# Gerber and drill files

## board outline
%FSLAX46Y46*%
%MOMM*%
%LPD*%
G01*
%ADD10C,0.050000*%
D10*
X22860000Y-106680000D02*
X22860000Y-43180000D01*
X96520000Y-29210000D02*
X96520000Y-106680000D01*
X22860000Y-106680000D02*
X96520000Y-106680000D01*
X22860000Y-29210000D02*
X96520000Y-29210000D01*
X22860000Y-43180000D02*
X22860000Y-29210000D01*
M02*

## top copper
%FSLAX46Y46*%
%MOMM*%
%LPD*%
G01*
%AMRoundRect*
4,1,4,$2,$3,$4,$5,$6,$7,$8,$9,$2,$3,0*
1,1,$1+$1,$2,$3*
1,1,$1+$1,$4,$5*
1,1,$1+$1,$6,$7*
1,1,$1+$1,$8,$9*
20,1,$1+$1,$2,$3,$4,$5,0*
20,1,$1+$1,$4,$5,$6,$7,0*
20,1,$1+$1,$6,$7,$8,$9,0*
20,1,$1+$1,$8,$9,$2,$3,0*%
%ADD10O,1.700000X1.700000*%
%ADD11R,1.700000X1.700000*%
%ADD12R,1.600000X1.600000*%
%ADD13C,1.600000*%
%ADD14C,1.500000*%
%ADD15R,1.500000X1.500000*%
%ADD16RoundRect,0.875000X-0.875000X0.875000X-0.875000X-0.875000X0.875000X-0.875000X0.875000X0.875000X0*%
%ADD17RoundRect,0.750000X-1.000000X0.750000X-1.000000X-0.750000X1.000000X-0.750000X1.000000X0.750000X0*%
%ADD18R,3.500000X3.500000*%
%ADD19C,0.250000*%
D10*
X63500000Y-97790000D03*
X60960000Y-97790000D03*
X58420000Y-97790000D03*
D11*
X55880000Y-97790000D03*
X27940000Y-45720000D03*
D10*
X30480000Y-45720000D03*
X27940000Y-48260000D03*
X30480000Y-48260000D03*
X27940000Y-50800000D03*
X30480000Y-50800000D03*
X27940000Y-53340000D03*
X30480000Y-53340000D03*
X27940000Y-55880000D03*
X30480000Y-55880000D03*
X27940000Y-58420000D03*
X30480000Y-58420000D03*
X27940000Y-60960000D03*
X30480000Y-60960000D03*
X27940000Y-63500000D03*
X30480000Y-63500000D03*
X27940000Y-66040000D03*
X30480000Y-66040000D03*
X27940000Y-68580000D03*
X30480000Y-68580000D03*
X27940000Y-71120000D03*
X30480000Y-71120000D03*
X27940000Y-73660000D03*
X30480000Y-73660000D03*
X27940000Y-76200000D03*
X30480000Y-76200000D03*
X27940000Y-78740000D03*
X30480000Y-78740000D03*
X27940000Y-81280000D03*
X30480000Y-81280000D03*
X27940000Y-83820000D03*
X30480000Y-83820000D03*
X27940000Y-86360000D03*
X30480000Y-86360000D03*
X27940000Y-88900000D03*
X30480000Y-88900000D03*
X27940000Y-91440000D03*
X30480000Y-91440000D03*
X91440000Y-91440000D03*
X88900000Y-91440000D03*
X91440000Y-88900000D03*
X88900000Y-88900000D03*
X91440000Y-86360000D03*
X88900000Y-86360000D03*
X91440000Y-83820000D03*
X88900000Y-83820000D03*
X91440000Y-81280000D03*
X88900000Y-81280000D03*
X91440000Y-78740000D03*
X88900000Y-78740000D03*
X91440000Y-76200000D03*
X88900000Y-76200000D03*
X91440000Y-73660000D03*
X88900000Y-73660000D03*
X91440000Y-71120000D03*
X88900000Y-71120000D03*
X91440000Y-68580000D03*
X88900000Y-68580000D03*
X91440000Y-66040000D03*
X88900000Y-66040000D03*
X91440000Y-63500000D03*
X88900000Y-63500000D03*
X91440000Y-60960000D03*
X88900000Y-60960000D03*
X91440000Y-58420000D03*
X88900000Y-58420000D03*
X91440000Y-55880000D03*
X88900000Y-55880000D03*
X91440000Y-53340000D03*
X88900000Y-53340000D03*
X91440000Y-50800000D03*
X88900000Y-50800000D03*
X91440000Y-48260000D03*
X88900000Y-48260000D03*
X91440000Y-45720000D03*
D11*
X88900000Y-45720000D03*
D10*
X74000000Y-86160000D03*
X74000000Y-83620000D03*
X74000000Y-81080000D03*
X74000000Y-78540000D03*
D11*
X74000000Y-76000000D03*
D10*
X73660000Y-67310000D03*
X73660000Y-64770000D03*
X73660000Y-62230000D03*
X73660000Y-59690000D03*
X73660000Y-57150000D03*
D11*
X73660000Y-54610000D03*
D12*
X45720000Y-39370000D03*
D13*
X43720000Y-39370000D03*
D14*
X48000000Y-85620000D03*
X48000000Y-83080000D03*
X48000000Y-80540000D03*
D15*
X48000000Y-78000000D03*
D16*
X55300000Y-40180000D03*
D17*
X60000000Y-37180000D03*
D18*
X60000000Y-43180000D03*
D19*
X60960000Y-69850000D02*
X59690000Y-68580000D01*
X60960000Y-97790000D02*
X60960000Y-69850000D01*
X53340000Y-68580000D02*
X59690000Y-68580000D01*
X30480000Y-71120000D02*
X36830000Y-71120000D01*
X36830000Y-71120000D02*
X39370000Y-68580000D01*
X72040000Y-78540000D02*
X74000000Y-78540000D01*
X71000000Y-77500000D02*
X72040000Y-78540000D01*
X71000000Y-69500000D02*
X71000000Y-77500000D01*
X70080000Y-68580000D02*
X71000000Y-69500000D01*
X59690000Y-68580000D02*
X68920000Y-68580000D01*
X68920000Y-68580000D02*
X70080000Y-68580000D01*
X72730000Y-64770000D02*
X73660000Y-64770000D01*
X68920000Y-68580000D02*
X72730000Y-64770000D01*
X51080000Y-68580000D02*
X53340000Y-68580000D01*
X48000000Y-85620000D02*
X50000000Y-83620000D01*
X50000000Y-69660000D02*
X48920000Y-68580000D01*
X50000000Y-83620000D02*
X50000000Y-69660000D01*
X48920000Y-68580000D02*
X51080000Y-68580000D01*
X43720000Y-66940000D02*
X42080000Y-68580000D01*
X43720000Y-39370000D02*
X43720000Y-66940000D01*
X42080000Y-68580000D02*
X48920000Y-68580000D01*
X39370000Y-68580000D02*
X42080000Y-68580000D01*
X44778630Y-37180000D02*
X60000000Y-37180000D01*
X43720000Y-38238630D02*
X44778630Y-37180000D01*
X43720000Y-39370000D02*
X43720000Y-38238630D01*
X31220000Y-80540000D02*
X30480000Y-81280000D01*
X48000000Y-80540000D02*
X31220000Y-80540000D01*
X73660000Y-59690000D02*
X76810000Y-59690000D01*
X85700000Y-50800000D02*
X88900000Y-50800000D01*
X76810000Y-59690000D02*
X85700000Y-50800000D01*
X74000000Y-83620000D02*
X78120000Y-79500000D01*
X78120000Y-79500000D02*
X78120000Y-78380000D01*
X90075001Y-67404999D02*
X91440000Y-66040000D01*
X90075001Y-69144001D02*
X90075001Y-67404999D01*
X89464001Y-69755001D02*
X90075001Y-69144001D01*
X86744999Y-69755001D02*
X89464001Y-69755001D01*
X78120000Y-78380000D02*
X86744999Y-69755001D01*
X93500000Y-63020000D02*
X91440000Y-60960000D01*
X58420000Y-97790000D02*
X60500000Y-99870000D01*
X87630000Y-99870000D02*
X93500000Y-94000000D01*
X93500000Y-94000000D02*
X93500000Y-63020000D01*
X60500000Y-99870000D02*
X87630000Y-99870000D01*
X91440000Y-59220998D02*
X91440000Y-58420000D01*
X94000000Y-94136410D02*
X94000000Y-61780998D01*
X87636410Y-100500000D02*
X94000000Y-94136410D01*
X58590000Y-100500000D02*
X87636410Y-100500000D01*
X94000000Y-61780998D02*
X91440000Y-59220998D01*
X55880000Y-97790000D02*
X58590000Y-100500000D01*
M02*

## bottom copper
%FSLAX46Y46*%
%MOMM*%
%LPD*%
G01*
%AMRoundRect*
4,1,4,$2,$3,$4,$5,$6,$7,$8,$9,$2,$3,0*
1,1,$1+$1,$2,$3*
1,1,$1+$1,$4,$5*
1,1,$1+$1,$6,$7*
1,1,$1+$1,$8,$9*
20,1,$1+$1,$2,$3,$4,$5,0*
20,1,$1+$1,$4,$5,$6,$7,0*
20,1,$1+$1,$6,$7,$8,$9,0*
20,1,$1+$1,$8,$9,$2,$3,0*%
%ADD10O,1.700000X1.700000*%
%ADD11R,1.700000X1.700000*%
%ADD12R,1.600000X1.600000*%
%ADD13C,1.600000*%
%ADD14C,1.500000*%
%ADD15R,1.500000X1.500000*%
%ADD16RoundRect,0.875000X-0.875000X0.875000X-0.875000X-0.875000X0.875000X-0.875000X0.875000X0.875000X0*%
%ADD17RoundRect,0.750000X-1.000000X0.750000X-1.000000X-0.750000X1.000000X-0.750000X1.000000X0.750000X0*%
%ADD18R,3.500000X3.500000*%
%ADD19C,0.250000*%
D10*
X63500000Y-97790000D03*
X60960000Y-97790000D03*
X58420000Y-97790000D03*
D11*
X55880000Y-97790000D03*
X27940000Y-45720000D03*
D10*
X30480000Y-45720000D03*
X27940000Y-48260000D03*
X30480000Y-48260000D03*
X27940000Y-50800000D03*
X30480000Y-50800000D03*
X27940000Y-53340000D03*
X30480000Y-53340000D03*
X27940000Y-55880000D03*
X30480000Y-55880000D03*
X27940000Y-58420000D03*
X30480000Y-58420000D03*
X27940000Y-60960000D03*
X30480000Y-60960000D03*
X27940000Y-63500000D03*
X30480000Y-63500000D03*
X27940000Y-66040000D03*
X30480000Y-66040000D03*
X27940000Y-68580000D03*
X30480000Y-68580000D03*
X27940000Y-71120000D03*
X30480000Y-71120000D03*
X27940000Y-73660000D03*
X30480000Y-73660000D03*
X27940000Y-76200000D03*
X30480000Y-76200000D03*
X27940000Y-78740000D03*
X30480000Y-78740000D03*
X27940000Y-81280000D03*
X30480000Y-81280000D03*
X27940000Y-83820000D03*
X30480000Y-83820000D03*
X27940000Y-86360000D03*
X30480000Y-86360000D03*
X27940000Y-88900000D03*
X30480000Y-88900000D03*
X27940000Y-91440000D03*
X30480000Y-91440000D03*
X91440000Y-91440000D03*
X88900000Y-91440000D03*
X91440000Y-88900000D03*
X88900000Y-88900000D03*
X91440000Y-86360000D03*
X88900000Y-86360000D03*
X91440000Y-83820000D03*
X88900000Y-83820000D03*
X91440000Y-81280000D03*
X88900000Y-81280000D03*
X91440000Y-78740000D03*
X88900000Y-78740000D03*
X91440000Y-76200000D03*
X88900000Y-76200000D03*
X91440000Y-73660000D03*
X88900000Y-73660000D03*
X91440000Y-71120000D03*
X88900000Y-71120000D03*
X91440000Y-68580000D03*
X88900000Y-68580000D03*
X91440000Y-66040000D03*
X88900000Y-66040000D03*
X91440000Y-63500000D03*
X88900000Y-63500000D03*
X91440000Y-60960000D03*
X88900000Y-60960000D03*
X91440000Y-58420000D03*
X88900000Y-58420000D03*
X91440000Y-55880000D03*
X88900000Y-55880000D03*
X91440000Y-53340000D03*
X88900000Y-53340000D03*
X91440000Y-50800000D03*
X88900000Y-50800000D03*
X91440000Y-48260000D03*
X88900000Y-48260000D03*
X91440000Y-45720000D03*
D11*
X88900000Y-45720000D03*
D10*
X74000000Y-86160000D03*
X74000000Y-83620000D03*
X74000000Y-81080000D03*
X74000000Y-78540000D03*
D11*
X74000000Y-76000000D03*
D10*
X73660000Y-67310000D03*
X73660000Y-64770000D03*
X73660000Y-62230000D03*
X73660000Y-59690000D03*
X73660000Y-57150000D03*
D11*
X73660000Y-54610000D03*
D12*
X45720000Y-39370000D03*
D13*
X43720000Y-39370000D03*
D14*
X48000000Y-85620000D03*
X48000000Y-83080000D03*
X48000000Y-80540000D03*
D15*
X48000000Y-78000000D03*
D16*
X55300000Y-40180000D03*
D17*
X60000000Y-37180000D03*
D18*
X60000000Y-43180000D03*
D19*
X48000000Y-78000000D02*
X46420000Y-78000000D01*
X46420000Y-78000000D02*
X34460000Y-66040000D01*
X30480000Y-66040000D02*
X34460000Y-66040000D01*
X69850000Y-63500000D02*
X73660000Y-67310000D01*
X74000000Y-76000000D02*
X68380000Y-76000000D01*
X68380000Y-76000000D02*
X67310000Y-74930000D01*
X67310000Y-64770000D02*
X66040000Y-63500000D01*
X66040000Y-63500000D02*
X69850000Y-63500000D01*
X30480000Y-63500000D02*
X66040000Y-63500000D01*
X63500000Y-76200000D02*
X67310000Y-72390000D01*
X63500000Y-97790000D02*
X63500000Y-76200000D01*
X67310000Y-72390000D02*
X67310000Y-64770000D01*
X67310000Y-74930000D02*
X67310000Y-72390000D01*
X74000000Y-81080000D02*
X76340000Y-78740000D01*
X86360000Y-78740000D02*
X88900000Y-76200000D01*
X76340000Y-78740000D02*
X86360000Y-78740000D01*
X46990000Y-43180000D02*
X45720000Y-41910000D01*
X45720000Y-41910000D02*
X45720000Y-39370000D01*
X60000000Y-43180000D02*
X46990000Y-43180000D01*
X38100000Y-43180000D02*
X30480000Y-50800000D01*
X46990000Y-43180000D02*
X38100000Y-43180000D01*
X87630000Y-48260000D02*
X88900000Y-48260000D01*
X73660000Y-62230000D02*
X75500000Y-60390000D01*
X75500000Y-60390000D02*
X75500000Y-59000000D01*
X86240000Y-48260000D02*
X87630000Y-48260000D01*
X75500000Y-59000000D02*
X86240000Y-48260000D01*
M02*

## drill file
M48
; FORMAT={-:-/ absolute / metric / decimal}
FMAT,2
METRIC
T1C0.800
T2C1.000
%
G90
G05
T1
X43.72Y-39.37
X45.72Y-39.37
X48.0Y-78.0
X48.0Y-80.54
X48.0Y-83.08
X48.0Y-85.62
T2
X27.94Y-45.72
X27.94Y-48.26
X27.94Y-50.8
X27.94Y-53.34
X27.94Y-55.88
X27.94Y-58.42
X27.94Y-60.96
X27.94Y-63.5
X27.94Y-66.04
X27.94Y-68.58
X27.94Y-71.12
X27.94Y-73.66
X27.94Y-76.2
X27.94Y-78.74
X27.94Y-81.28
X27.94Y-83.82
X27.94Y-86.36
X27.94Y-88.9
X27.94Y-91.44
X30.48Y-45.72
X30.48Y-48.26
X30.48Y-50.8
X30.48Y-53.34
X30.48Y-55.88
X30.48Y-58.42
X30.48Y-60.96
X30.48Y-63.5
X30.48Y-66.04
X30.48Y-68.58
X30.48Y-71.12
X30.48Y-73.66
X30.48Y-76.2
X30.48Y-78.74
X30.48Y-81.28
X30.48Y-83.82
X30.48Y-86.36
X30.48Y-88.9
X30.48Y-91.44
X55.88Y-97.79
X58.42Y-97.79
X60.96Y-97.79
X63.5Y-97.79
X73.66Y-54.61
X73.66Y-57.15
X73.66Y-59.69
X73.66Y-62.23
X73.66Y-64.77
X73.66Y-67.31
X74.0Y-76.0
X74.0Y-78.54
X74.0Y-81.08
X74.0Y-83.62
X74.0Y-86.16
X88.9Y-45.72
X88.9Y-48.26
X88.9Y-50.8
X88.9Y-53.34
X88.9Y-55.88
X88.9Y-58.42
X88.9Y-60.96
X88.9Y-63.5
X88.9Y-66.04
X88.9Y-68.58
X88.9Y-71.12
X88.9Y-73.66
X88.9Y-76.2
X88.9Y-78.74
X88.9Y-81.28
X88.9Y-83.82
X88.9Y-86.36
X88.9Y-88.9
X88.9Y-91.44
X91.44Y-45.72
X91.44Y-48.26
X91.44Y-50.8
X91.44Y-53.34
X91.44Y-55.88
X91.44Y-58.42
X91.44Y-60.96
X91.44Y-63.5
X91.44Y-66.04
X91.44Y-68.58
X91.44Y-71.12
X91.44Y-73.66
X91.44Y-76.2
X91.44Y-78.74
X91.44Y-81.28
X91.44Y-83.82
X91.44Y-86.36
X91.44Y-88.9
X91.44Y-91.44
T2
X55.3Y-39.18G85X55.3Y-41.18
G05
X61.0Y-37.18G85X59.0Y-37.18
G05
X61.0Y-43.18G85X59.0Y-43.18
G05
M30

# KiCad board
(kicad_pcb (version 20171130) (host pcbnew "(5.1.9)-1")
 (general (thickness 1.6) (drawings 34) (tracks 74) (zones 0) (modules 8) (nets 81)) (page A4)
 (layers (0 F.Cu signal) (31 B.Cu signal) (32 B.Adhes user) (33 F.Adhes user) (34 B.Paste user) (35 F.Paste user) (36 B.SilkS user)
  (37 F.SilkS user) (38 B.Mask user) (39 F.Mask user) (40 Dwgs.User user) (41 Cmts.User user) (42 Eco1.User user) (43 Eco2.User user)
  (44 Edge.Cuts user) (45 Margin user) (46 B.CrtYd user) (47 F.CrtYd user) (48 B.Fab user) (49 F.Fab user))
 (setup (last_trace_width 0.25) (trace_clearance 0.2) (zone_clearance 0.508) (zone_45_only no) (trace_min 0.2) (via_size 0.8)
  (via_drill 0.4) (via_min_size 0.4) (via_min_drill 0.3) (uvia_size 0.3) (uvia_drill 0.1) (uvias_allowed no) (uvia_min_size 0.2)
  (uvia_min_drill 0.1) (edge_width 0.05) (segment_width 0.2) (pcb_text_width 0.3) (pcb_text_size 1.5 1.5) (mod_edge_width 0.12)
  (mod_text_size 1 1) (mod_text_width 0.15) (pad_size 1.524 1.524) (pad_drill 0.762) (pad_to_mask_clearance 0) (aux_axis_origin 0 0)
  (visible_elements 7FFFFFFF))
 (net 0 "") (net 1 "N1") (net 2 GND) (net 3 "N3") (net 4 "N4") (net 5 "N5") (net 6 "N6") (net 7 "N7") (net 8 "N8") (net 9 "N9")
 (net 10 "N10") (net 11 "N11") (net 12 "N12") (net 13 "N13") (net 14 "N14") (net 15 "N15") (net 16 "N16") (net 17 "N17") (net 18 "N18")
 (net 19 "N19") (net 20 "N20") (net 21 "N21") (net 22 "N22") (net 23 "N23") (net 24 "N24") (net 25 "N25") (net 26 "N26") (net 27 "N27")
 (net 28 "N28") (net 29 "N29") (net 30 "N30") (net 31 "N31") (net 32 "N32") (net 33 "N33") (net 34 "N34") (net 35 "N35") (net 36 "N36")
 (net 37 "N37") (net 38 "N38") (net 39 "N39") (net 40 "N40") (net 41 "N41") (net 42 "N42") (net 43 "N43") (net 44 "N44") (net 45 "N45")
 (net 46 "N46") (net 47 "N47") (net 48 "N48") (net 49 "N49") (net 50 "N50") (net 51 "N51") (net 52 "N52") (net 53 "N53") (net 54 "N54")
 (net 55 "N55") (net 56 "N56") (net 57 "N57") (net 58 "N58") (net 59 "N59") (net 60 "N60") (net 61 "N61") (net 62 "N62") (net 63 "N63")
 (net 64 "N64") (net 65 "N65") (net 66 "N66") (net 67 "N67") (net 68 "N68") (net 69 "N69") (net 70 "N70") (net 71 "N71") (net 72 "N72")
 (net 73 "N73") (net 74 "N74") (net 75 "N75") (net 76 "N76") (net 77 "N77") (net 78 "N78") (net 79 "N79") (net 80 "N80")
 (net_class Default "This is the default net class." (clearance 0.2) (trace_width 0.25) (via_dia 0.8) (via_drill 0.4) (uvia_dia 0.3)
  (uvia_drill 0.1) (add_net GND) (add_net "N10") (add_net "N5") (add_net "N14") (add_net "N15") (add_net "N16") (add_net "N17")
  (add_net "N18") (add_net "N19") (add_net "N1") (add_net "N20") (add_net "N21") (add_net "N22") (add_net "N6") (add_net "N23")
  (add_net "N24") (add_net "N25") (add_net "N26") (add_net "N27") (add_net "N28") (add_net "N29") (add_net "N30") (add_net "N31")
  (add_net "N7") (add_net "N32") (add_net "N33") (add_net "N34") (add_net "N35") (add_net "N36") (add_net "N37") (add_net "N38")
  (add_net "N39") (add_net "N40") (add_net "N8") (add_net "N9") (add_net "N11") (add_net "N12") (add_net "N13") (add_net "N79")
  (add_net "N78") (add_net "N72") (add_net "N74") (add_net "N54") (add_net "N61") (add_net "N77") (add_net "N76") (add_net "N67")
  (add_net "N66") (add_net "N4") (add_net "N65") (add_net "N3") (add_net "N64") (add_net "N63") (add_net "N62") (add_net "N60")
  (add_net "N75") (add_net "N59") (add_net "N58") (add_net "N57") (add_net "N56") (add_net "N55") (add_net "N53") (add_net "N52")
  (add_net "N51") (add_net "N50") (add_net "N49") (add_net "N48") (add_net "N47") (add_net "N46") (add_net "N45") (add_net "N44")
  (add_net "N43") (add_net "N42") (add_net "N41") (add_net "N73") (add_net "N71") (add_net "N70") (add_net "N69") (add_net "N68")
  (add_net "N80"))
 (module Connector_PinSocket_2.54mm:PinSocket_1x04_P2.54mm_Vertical (layer F.Cu) (at 55.88 97.79 90)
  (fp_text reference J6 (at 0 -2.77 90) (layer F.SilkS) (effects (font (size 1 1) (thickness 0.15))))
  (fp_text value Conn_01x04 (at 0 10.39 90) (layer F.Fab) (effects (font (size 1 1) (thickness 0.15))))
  (pad 4 thru_hole oval (at 0 7.62 90) (size 1.7 1.7) (drill 1) (layers *.Cu *.Mask) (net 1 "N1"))
  (pad 3 thru_hole oval (at 0 5.08 90) (size 1.7 1.7) (drill 1) (layers *.Cu *.Mask) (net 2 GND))
  (pad 2 thru_hole oval (at 0 2.54 90) (size 1.7 1.7) (drill 1) (layers *.Cu *.Mask) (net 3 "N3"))
  (pad 1 thru_hole rect (at 0 0 90) (size 1.7 1.7) (drill 1) (layers *.Cu *.Mask) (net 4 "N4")))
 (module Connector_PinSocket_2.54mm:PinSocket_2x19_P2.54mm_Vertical (layer B.Cu) (at 27.94 45.72 180)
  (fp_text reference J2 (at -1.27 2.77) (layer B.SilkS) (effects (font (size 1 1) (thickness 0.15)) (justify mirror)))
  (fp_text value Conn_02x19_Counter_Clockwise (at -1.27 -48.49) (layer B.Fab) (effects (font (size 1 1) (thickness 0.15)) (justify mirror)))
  (pad 1 thru_hole rect (at 0 0 180) (size 1.7 1.7) (drill 1) (layers *.Cu *.Mask) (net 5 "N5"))
  (pad 2 thru_hole oval (at -2.54 0 180) (size 1.7 1.7) (drill 1) (layers *.Cu *.Mask) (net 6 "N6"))
  (pad 3 thru_hole oval (at 0 -2.54 180) (size 1.7 1.7) (drill 1) (layers *.Cu *.Mask) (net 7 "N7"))
  (pad 4 thru_hole oval (at -2.54 -2.54 180) (size 1.7 1.7) (drill 1) (layers *.Cu *.Mask) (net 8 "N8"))
  (pad 5 thru_hole oval (at 0 -5.08 180) (size 1.7 1.7) (drill 1) (layers *.Cu *.Mask) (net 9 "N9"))
  (pad 6 thru_hole oval (at -2.54 -5.08 180) (size 1.7 1.7) (drill 1) (layers *.Cu *.Mask) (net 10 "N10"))
  (pad 7 thru_hole oval (at 0 -7.62 180) (size 1.7 1.7) (drill 1) (layers *.Cu *.Mask) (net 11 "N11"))
  (pad 8 thru_hole oval (at -2.54 -7.62 180) (size 1.7 1.7) (drill 1) (layers *.Cu *.Mask) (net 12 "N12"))
  (pad 9 thru_hole oval (at 0 -10.16 180) (size 1.7 1.7) (drill 1) (layers *.Cu *.Mask) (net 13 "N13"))
  (pad 10 thru_hole oval (at -2.54 -10.16 180) (size 1.7 1.7) (drill 1) (layers *.Cu *.Mask) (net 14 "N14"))
  (pad 11 thru_hole oval (at 0 -12.7 180) (size 1.7 1.7) (drill 1) (layers *.Cu *.Mask) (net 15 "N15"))
  (pad 12 thru_hole oval (at -2.54 -12.7 180) (size 1.7 1.7) (drill 1) (layers *.Cu *.Mask) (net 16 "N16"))
  (pad 13 thru_hole oval (at 0 -15.24 180) (size 1.7 1.7) (drill 1) (layers *.Cu *.Mask) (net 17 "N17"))
  (pad 14 thru_hole oval (at -2.54 -15.24 180) (size 1.7 1.7) (drill 1) (layers *.Cu *.Mask) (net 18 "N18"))
  (pad 15 thru_hole oval (at 0 -17.78 180) (size 1.7 1.7) (drill 1) (layers *.Cu *.Mask) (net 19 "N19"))
  (pad 16 thru_hole oval (at -2.54 -17.78 180) (size 1.7 1.7) (drill 1) (layers *.Cu *.Mask) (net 1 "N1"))
  (pad 17 thru_hole oval (at 0 -20.32 180) (size 1.7 1.7) (drill 1) (layers *.Cu *.Mask) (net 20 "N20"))
  (pad 18 thru_hole oval (at -2.54 -20.32 180) (size 1.7 1.7) (drill 1) (layers *.Cu *.Mask) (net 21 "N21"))
  (pad 19 thru_hole oval (at 0 -22.86 180) (size 1.7 1.7) (drill 1) (layers *.Cu *.Mask) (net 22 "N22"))
  (pad 20 thru_hole oval (at -2.54 -22.86 180) (size 1.7 1.7) (drill 1) (layers *.Cu *.Mask) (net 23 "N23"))
  (pad 21 thru_hole oval (at 0 -25.4 180) (size 1.7 1.7) (drill 1) (layers *.Cu *.Mask) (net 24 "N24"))
  (pad 22 thru_hole oval (at -2.54 -25.4 180) (size 1.7 1.7) (drill 1) (layers *.Cu *.Mask) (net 2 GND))
  (pad 23 thru_hole oval (at 0 -27.94 180) (size 1.7 1.7) (drill 1) (layers *.Cu *.Mask) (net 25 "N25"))
  (pad 24 thru_hole oval (at -2.54 -27.94 180) (size 1.7 1.7) (drill 1) (layers *.Cu *.Mask) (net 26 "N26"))
  (pad 25 thru_hole oval (at 0 -30.48 180) (size 1.7 1.7) (drill 1) (layers *.Cu *.Mask) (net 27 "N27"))
  (pad 26 thru_hole oval (at -2.54 -30.48 180) (size 1.7 1.7) (drill 1) (layers *.Cu *.Mask) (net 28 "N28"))
  (pad 27 thru_hole oval (at 0 -33.02 180) (size 1.7 1.7) (drill 1) (layers *.Cu *.Mask) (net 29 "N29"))
  (pad 28 thru_hole oval (at -2.54 -33.02 180) (size 1.7 1.7) (drill 1) (layers *.Cu *.Mask) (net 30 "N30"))
  (pad 29 thru_hole oval (at 0 -35.56 180) (size 1.7 1.7) (drill 1) (layers *.Cu *.Mask) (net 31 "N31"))
  (pad 30 thru_hole oval (at -2.54 -35.56 180) (size 1.7 1.7) (drill 1) (layers *.Cu *.Mask) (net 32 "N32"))
  (pad 31 thru_hole oval (at 0 -38.1 180) (size 1.7 1.7) (drill 1) (layers *.Cu *.Mask) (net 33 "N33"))
  (pad 32 thru_hole oval (at -2.54 -38.1 180) (size 1.7 1.7) (drill 1) (layers *.Cu *.Mask) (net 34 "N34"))
  (pad 33 thru_hole oval (at 0 -40.64 180) (size 1.7 1.7) (drill 1) (layers *.Cu *.Mask) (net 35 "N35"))
  (pad 34 thru_hole oval (at -2.54 -40.64 180) (size 1.7 1.7) (drill 1) (layers *.Cu *.Mask) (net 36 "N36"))
  (pad 35 thru_hole oval (at 0 -43.18 180) (size 1.7 1.7) (drill 1) (layers *.Cu *.Mask) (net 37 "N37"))
  (pad 36 thru_hole oval (at -2.54 -43.18 180) (size 1.7 1.7) (drill 1) (layers *.Cu *.Mask) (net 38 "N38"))
  (pad 37 thru_hole oval (at 0 -45.72 180) (size 1.7 1.7) (drill 1) (layers *.Cu *.Mask) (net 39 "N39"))
  (pad 38 thru_hole oval (at -2.54 -45.72 180) (size 1.7 1.7) (drill 1) (layers *.Cu *.Mask) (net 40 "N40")))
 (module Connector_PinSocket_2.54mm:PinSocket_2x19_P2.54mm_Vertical (layer B.Cu) (at 88.9 45.72 180)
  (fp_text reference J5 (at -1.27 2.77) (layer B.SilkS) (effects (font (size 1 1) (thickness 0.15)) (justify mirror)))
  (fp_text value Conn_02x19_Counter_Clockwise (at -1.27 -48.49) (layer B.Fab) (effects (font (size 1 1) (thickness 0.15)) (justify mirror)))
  (pad 38 thru_hole oval (at -2.54 -45.72 180) (size 1.7 1.7) (drill 1) (layers *.Cu *.Mask) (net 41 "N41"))
  (pad 37 thru_hole oval (at 0 -45.72 180) (size 1.7 1.7) (drill 1) (layers *.Cu *.Mask) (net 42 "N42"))
  (pad 36 thru_hole oval (at -2.54 -43.18 180) (size 1.7 1.7) (drill 1) (layers *.Cu *.Mask) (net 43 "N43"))
  (pad 35 thru_hole oval (at 0 -43.18 180) (size 1.7 1.7) (drill 1) (layers *.Cu *.Mask) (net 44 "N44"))
  (pad 34 thru_hole oval (at -2.54 -40.64 180) (size 1.7 1.7) (drill 1) (layers *.Cu *.Mask) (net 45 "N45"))
  (pad 33 thru_hole oval (at 0 -40.64 180) (size 1.7 1.7) (drill 1) (layers *.Cu *.Mask) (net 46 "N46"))
  (pad 32 thru_hole oval (at -2.54 -38.1 180) (size 1.7 1.7) (drill 1) (layers *.Cu *.Mask) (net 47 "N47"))
  (pad 31 thru_hole oval (at 0 -38.1 180) (size 1.7 1.7) (drill 1) (layers *.Cu *.Mask) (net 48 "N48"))
  (pad 30 thru_hole oval (at -2.54 -35.56 180) (size 1.7 1.7) (drill 1) (layers *.Cu *.Mask) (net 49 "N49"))
  (pad 29 thru_hole oval (at 0 -35.56 180) (size 1.7 1.7) (drill 1) (layers *.Cu *.Mask) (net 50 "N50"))
  (pad 28 thru_hole oval (at -2.54 -33.02 180) (size 1.7 1.7) (drill 1) (layers *.Cu *.Mask) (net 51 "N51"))
  (pad 27 thru_hole oval (at 0 -33.02 180) (size 1.7 1.7) (drill 1) (layers *.Cu *.Mask) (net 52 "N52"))
  (pad 26 thru_hole oval (at -2.54 -30.48 180) (size 1.7 1.7) (drill 1) (layers *.Cu *.Mask) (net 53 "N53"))
  (pad 25 thru_hole oval (at 0 -30.48 180) (size 1.7 1.7) (drill 1) (layers *.Cu *.Mask) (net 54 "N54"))
  (pad 24 thru_hole oval (at -2.54 -27.94 180) (size 1.7 1.7) (drill 1) (layers *.Cu *.Mask) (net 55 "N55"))
  (pad 23 thru_hole oval (at 0 -27.94 180) (size 1.7 1.7) (drill 1) (layers *.Cu *.Mask) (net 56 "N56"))
  (pad 22 thru_hole oval (at -2.54 -25.4 180) (size 1.7 1.7) (drill 1) (layers *.Cu *.Mask) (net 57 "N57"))
  (pad 21 thru_hole oval (at 0 -25.4 180) (size 1.7 1.7) (drill 1) (layers *.Cu *.Mask) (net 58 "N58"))
  (pad 20 thru_hole oval (at -2.54 -22.86 180) (size 1.7 1.7) (drill 1) (layers *.Cu *.Mask) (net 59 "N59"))
  (pad 19 thru_hole oval (at 0 -22.86 180) (size 1.7 1.7) (drill 1) (layers *.Cu *.Mask) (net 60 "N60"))
  (pad 18 thru_hole oval (at -2.54 -20.32 180) (size 1.7 1.7) (drill 1) (layers *.Cu *.Mask) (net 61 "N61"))
  (pad 17 thru_hole oval (at 0 -20.32 180) (size 1.7 1.7) (drill 1) (layers *.Cu *.Mask) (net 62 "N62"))
  (pad 16 thru_hole oval (at -2.54 -17.78 180) (size 1.7 1.7) (drill 1) (layers *.Cu *.Mask) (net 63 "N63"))
  (pad 15 thru_hole oval (at 0 -17.78 180) (size 1.7 1.7) (drill 1) (layers *.Cu *.Mask) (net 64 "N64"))
  (pad 14 thru_hole oval (at -2.54 -15.24 180) (size 1.7 1.7) (drill 1) (layers *.Cu *.Mask) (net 3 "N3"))
  (pad 13 thru_hole oval (at 0 -15.24 180) (size 1.7 1.7) (drill 1) (layers *.Cu *.Mask) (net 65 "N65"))
  (pad 12 thru_hole oval (at -2.54 -12.7 180) (size 1.7 1.7) (drill 1) (layers *.Cu *.Mask) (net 4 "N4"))
  (pad 11 thru_hole oval (at 0 -12.7 180) (size 1.7 1.7) (drill 1) (layers *.Cu *.Mask) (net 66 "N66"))
  (pad 10 thru_hole oval (at -2.54 -10.16 180) (size 1.7 1.7) (drill 1) (layers *.Cu *.Mask) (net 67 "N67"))
  (pad 9 thru_hole oval (at 0 -10.16 180) (size 1.7 1.7) (drill 1) (layers *.Cu *.Mask) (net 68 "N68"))
  (pad 8 thru_hole oval (at -2.54 -7.62 180) (size 1.7 1.7) (drill 1) (layers *.Cu *.Mask) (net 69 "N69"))
  (pad 7 thru_hole oval (at 0 -7.62 180) (size 1.7 1.7) (drill 1) (layers *.Cu *.Mask) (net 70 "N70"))
  (pad 6 thru_hole oval (at -2.54 -5.08 180) (size 1.7 1.7) (drill 1) (layers *.Cu *.Mask) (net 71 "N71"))
  (pad 5 thru_hole oval (at 0 -5.08 180) (size 1.7 1.7) (drill 1) (layers *.Cu *.Mask) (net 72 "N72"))
  (pad 4 thru_hole oval (at -2.54 -2.54 180) (size 1.7 1.7) (drill 1) (layers *.Cu *.Mask) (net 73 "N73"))
  (pad 3 thru_hole oval (at 0 -2.54 180) (size 1.7 1.7) (drill 1) (layers *.Cu *.Mask) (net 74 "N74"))
  (pad 2 thru_hole oval (at -2.54 0 180) (size 1.7 1.7) (drill 1) (layers *.Cu *.Mask) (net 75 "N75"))
  (pad 1 thru_hole rect (at 0 0 180) (size 1.7 1.7) (drill 1) (layers *.Cu *.Mask) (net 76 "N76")))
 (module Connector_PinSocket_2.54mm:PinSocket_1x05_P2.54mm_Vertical (layer F.Cu) (at 74 76)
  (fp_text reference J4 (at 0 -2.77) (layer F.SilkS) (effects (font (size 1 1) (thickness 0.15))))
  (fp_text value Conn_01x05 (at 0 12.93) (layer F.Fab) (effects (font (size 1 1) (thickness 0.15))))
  (pad 5 thru_hole oval (at 0 10.16) (size 1.7 1.7) (drill 1) (layers *.Cu *.Mask) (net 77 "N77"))
  (pad 4 thru_hole oval (at 0 7.62) (size 1.7 1.7) (drill 1) (layers *.Cu *.Mask) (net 61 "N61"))
  (pad 3 thru_hole oval (at 0 5.08) (size 1.7 1.7) (drill 1) (layers *.Cu *.Mask) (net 54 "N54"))
  (pad 2 thru_hole oval (at 0 2.54) (size 1.7 1.7) (drill 1) (layers *.Cu *.Mask) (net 2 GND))
  (pad 1 thru_hole rect (at 0 0) (size 1.7 1.7) (drill 1) (layers *.Cu *.Mask) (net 1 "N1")))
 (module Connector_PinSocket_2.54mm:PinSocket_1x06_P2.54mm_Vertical (layer F.Cu) (at 73.66 54.61)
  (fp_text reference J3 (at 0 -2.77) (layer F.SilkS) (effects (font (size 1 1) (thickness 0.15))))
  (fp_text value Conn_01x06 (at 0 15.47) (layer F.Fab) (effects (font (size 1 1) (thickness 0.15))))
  (pad 6 thru_hole oval (at 0 12.7) (size 1.7 1.7) (drill 1) (layers *.Cu *.Mask) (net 1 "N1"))
  (pad 5 thru_hole oval (at 0 10.16) (size 1.7 1.7) (drill 1) (layers *.Cu *.Mask) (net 2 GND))
  (pad 4 thru_hole oval (at 0 7.62) (size 1.7 1.7) (drill 1) (layers *.Cu *.Mask) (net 74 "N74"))
  (pad 3 thru_hole oval (at 0 5.08) (size 1.7 1.7) (drill 1) (layers *.Cu *.Mask) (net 72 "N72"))
  (pad 2 thru_hole oval (at 0 2.54) (size 1.7 1.7) (drill 1) (layers *.Cu *.Mask) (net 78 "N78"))
  (pad 1 thru_hole rect (at 0 0) (size 1.7 1.7) (drill 1) (layers *.Cu *.Mask) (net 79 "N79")))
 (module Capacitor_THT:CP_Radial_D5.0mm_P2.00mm (layer F.Cu) (at 45.72 39.37 180)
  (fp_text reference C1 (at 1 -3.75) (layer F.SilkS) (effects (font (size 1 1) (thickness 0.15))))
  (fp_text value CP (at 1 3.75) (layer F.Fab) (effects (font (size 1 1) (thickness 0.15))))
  (pad 1 thru_hole rect (at 0 0 180) (size 1.6 1.6) (drill 0.8) (layers *.Cu *.Mask) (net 10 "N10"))
  (pad 2 thru_hole circle (at 2 0 180) (size 1.6 1.6) (drill 0.8) (layers *.Cu *.Mask) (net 2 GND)))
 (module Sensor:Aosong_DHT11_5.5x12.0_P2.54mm (layer F.Cu) (at 48 78)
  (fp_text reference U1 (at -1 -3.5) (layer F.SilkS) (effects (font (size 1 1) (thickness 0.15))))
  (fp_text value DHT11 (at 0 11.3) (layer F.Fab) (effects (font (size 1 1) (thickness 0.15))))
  (pad 4 thru_hole circle (at 0 7.62) (size 1.5 1.5) (drill 0.8) (layers *.Cu *.Mask) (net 2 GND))
  (pad 3 thru_hole circle (at 0 5.08) (size 1.5 1.5) (drill 0.8) (layers *.Cu *.Mask) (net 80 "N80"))
  (pad 2 thru_hole circle (at 0 2.54) (size 1.5 1.5) (drill 0.8) (layers *.Cu *.Mask) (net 32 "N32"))
  (pad 1 thru_hole rect (at 0 0) (size 1.5 1.5) (drill 0.8) (layers *.Cu *.Mask) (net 21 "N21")))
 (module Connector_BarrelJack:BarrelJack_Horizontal (layer F.Cu) (at 60 43.18 270)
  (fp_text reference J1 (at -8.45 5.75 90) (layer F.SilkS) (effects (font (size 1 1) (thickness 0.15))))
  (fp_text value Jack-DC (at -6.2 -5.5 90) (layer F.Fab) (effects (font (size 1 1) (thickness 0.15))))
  (pad 3 thru_hole roundrect (at -3 4.7 270) (size 3.5 3.5) (drill oval 3 1) (layers *.Cu *.Mask) (roundrect_rratio 0.25))
  (pad 2 thru_hole roundrect (at -6 0 270) (size 3 3.5) (drill oval 1 3) (layers *.Cu *.Mask) (roundrect_rratio 0.25) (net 2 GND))
  (pad 1 thru_hole rect (at 0 0 270) (size 3.5 3.5) (drill oval 1 3) (layers *.Cu *.Mask) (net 10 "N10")))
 (gr_line (start 22.86 106.68) (end 22.86 43.18) (layer Edge.Cuts) (width 0.05))
 (gr_line (start 96.52 29.21) (end 96.52 106.68) (layer Edge.Cuts) (width 0.05))
 (gr_line (start 22.86 106.68) (end 96.52 106.68) (layer Edge.Cuts) (width 0.05))
 (gr_line (start 22.86 29.21) (end 96.52 29.21) (layer Edge.Cuts) (width 0.05))
 (gr_line (start 22.86 43.18) (end 22.86 29.21) (layer Edge.Cuts) (width 0.05))
 (segment (start 60.96 69.85) (end 59.69 68.58) (width 0.25) (layer F.Cu) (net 2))
 (segment (start 60.96 97.79) (end 60.96 69.85) (width 0.25) (layer F.Cu) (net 2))
 (segment (start 53.34 68.58) (end 59.69 68.58) (width 0.25) (layer F.Cu) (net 2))
 (segment (start 30.48 71.12) (end 36.83 71.12) (width 0.25) (layer F.Cu) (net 2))
 (segment (start 36.83 71.12) (end 39.37 68.58) (width 0.25) (layer F.Cu) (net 2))
 (segment (start 72.04 78.54) (end 74 78.54) (width 0.25) (layer F.Cu) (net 2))
 (segment (start 71 77.5) (end 72.04 78.54) (width 0.25) (layer F.Cu) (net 2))
 (segment (start 71 69.5) (end 71 77.5) (width 0.25) (layer F.Cu) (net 2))
 (segment (start 70.08 68.58) (end 71 69.5) (width 0.25) (layer F.Cu) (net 2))
 (segment (start 59.69 68.58) (end 68.92 68.58) (width 0.25) (layer F.Cu) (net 2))
 (segment (start 68.92 68.58) (end 70.08 68.58) (width 0.25) (layer F.Cu) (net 2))
 (segment (start 72.73 64.77) (end 73.66 64.77) (width 0.25) (layer F.Cu) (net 2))
 (segment (start 68.92 68.58) (end 72.73 64.77) (width 0.25) (layer F.Cu) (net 2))
 (segment (start 51.08 68.58) (end 53.34 68.58) (width 0.25) (layer F.Cu) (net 2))
 (segment (start 48 85.62) (end 50 83.62) (width 0.25) (layer F.Cu) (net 2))
 (segment (start 50 69.66) (end 48.92 68.58) (width 0.25) (layer F.Cu) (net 2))
 (segment (start 50 83.62) (end 50 69.66) (width 0.25) (layer F.Cu) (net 2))
 (segment (start 48.92 68.58) (end 51.08 68.58) (width 0.25) (layer F.Cu) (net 2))
 (segment (start 43.72 66.94) (end 42.08 68.58) (width 0.25) (layer F.Cu) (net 2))
 (segment (start 43.72 39.37) (end 43.72 66.94) (width 0.25) (layer F.Cu) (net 2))
 (segment (start 42.08 68.58) (end 48.92 68.58) (width 0.25) (layer F.Cu) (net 2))
 (segment (start 39.37 68.58) (end 42.08 68.58) (width 0.25) (layer F.Cu) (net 2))
 (segment (start 44.77863 37.18) (end 60 37.18) (width 0.25) (layer F.Cu) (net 2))
 (segment (start 43.72 38.23863) (end 44.77863 37.18) (width 0.25) (layer F.Cu) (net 2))
 (segment (start 43.72 39.37) (end 43.72 38.23863) (width 0.25) (layer F.Cu) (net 2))
 (segment (start 31.22 80.54) (end 30.48 81.28) (width 0.25) (layer F.Cu) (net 32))
 (segment (start 48 80.54) (end 31.22 80.54) (width 0.25) (layer F.Cu) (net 32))
 (segment (start 48 78) (end 46.42 78) (width 0.25) (layer B.Cu) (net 21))
 (segment (start 46.42 78) (end 34.46 66.04) (width 0.25) (layer B.Cu) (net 21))
 (segment (start 30.48 66.04) (end 34.46 66.04) (width 0.25) (layer B.Cu) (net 21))
 (segment (start 69.85 63.5) (end 73.66 67.31) (width 0.25) (layer B.Cu) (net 1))
 (segment (start 74 76) (end 68.38 76) (width 0.25) (layer B.Cu) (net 1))
 (segment (start 68.38 76) (end 67.31 74.93) (width 0.25) (layer B.Cu) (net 1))
 (segment (start 67.31 64.77) (end 66.04 63.5) (width 0.25) (layer B.Cu) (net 1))
 (segment (start 66.04 63.5) (end 69.85 63.5) (width 0.25) (layer B.Cu) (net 1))
 (segment (start 30.48 63.5) (end 66.04 63.5) (width 0.25) (layer B.Cu) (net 1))
 (segment (start 63.5 76.2) (end 67.31 72.39) (width 0.25) (layer B.Cu) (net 1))
 (segment (start 63.5 97.79) (end 63.5 76.2) (width 0.25) (layer B.Cu) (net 1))
 (segment (start 67.31 72.39) (end 67.31 64.77) (width 0.25) (layer B.Cu) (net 1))
 (segment (start 67.31 74.93) (end 67.31 72.39) (width 0.25) (layer B.Cu) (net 1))
 (segment (start 73.66 59.69) (end 76.81 59.69) (width 0.25) (layer F.Cu) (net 72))
 (segment (start 85.7 50.8) (end 88.9 50.8) (width 0.25) (layer F.Cu) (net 72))
 (segment (start 76.81 59.69) (end 85.7 50.8) (width 0.25) (layer F.Cu) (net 72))
 (segment (start 74 83.62) (end 78.12 79.5) (width 0.25) (layer F.Cu) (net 61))
 (segment (start 78.12 79.5) (end 78.12 78.38) (width 0.25) (layer F.Cu) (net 61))
 (segment (start 90.075001 67.404999) (end 91.44 66.04) (width 0.25) (layer F.Cu) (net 61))
 (segment (start 90.075001 69.144001) (end 90.075001 67.404999) (width 0.25) (layer F.Cu) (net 61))
 (segment (start 89.464001 69.755001) (end 90.075001 69.144001) (width 0.25) (layer F.Cu) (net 61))
 (segment (start 86.744999 69.755001) (end 89.464001 69.755001) (width 0.25) (layer F.Cu) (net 61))
 (segment (start 78.12 78.38) (end 86.744999 69.755001) (width 0.25) (layer F.Cu) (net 61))
 (segment (start 74 81.08) (end 76.34 78.74) (width 0.25) (layer B.Cu) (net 54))
 (segment (start 86.36 78.74) (end 88.9 76.2) (width 0.25) (layer B.Cu) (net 54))
 (segment (start 76.34 78.74) (end 86.36 78.74) (width 0.25) (layer B.Cu) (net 54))
 (segment (start 93.5 63.02) (end 91.44 60.96) (width 0.25) (layer F.Cu) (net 3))
 (segment (start 58.42 97.79) (end 60.5 99.87) (width 0.25) (layer F.Cu) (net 3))
 (segment (start 87.63 99.87) (end 93.5 94) (width 0.25) (layer F.Cu) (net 3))
 (segment (start 93.5 94) (end 93.5 63.02) (width 0.25) (layer F.Cu) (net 3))
 (segment (start 60.5 99.87) (end 87.63 99.87) (width 0.25) (layer F.Cu) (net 3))
 (segment (start 91.44 59.220998) (end 91.44 58.42) (width 0.25) (layer F.Cu) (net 4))
 (segment (start 94 94.13641) (end 94 61.780998) (width 0.25) (layer F.Cu) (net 4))
 (segment (start 87.63641 100.5) (end 94 94.13641) (width 0.25) (layer F.Cu) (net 4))
 (segment (start 58.59 100.5) (end 87.63641 100.5) (width 0.25) (layer F.Cu) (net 4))
 (segment (start 94 61.780998) (end 91.44 59.220998) (width 0.25) (layer F.Cu) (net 4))
 (segment (start 55.88 97.79) (end 58.59 100.5) (width 0.25) (layer F.Cu) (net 4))
 (segment (start 46.99 43.18) (end 45.72 41.91) (width 0.25) (layer B.Cu) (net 10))
 (segment (start 45.72 41.91) (end 45.72 39.37) (width 0.25) (layer B.Cu) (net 10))
 (segment (start 60 43.18) (end 46.99 43.18) (width 0.25) (layer B.Cu) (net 10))
 (segment (start 38.1 43.18) (end 30.48 50.8) (width 0.25) (layer B.Cu) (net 10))
 (segment (start 46.99 43.18) (end 38.1 43.18) (width 0.25) (layer B.Cu) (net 10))
 (segment (start 87.63 48.26) (end 88.9 48.26) (width 0.25) (layer B.Cu) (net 74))
 (segment (start 73.66 62.23) (end 75.5 60.39) (width 0.25) (layer B.Cu) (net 74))
 (segment (start 75.5 60.39) (end 75.5 59) (width 0.25) (layer B.Cu) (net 74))
 (segment (start 86.24 48.26) (end 87.63 48.26) (width 0.25) (layer B.Cu) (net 74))
 (segment (start 75.5 59) (end 86.24 48.26) (width 0.25) (layer B.Cu) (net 74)))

